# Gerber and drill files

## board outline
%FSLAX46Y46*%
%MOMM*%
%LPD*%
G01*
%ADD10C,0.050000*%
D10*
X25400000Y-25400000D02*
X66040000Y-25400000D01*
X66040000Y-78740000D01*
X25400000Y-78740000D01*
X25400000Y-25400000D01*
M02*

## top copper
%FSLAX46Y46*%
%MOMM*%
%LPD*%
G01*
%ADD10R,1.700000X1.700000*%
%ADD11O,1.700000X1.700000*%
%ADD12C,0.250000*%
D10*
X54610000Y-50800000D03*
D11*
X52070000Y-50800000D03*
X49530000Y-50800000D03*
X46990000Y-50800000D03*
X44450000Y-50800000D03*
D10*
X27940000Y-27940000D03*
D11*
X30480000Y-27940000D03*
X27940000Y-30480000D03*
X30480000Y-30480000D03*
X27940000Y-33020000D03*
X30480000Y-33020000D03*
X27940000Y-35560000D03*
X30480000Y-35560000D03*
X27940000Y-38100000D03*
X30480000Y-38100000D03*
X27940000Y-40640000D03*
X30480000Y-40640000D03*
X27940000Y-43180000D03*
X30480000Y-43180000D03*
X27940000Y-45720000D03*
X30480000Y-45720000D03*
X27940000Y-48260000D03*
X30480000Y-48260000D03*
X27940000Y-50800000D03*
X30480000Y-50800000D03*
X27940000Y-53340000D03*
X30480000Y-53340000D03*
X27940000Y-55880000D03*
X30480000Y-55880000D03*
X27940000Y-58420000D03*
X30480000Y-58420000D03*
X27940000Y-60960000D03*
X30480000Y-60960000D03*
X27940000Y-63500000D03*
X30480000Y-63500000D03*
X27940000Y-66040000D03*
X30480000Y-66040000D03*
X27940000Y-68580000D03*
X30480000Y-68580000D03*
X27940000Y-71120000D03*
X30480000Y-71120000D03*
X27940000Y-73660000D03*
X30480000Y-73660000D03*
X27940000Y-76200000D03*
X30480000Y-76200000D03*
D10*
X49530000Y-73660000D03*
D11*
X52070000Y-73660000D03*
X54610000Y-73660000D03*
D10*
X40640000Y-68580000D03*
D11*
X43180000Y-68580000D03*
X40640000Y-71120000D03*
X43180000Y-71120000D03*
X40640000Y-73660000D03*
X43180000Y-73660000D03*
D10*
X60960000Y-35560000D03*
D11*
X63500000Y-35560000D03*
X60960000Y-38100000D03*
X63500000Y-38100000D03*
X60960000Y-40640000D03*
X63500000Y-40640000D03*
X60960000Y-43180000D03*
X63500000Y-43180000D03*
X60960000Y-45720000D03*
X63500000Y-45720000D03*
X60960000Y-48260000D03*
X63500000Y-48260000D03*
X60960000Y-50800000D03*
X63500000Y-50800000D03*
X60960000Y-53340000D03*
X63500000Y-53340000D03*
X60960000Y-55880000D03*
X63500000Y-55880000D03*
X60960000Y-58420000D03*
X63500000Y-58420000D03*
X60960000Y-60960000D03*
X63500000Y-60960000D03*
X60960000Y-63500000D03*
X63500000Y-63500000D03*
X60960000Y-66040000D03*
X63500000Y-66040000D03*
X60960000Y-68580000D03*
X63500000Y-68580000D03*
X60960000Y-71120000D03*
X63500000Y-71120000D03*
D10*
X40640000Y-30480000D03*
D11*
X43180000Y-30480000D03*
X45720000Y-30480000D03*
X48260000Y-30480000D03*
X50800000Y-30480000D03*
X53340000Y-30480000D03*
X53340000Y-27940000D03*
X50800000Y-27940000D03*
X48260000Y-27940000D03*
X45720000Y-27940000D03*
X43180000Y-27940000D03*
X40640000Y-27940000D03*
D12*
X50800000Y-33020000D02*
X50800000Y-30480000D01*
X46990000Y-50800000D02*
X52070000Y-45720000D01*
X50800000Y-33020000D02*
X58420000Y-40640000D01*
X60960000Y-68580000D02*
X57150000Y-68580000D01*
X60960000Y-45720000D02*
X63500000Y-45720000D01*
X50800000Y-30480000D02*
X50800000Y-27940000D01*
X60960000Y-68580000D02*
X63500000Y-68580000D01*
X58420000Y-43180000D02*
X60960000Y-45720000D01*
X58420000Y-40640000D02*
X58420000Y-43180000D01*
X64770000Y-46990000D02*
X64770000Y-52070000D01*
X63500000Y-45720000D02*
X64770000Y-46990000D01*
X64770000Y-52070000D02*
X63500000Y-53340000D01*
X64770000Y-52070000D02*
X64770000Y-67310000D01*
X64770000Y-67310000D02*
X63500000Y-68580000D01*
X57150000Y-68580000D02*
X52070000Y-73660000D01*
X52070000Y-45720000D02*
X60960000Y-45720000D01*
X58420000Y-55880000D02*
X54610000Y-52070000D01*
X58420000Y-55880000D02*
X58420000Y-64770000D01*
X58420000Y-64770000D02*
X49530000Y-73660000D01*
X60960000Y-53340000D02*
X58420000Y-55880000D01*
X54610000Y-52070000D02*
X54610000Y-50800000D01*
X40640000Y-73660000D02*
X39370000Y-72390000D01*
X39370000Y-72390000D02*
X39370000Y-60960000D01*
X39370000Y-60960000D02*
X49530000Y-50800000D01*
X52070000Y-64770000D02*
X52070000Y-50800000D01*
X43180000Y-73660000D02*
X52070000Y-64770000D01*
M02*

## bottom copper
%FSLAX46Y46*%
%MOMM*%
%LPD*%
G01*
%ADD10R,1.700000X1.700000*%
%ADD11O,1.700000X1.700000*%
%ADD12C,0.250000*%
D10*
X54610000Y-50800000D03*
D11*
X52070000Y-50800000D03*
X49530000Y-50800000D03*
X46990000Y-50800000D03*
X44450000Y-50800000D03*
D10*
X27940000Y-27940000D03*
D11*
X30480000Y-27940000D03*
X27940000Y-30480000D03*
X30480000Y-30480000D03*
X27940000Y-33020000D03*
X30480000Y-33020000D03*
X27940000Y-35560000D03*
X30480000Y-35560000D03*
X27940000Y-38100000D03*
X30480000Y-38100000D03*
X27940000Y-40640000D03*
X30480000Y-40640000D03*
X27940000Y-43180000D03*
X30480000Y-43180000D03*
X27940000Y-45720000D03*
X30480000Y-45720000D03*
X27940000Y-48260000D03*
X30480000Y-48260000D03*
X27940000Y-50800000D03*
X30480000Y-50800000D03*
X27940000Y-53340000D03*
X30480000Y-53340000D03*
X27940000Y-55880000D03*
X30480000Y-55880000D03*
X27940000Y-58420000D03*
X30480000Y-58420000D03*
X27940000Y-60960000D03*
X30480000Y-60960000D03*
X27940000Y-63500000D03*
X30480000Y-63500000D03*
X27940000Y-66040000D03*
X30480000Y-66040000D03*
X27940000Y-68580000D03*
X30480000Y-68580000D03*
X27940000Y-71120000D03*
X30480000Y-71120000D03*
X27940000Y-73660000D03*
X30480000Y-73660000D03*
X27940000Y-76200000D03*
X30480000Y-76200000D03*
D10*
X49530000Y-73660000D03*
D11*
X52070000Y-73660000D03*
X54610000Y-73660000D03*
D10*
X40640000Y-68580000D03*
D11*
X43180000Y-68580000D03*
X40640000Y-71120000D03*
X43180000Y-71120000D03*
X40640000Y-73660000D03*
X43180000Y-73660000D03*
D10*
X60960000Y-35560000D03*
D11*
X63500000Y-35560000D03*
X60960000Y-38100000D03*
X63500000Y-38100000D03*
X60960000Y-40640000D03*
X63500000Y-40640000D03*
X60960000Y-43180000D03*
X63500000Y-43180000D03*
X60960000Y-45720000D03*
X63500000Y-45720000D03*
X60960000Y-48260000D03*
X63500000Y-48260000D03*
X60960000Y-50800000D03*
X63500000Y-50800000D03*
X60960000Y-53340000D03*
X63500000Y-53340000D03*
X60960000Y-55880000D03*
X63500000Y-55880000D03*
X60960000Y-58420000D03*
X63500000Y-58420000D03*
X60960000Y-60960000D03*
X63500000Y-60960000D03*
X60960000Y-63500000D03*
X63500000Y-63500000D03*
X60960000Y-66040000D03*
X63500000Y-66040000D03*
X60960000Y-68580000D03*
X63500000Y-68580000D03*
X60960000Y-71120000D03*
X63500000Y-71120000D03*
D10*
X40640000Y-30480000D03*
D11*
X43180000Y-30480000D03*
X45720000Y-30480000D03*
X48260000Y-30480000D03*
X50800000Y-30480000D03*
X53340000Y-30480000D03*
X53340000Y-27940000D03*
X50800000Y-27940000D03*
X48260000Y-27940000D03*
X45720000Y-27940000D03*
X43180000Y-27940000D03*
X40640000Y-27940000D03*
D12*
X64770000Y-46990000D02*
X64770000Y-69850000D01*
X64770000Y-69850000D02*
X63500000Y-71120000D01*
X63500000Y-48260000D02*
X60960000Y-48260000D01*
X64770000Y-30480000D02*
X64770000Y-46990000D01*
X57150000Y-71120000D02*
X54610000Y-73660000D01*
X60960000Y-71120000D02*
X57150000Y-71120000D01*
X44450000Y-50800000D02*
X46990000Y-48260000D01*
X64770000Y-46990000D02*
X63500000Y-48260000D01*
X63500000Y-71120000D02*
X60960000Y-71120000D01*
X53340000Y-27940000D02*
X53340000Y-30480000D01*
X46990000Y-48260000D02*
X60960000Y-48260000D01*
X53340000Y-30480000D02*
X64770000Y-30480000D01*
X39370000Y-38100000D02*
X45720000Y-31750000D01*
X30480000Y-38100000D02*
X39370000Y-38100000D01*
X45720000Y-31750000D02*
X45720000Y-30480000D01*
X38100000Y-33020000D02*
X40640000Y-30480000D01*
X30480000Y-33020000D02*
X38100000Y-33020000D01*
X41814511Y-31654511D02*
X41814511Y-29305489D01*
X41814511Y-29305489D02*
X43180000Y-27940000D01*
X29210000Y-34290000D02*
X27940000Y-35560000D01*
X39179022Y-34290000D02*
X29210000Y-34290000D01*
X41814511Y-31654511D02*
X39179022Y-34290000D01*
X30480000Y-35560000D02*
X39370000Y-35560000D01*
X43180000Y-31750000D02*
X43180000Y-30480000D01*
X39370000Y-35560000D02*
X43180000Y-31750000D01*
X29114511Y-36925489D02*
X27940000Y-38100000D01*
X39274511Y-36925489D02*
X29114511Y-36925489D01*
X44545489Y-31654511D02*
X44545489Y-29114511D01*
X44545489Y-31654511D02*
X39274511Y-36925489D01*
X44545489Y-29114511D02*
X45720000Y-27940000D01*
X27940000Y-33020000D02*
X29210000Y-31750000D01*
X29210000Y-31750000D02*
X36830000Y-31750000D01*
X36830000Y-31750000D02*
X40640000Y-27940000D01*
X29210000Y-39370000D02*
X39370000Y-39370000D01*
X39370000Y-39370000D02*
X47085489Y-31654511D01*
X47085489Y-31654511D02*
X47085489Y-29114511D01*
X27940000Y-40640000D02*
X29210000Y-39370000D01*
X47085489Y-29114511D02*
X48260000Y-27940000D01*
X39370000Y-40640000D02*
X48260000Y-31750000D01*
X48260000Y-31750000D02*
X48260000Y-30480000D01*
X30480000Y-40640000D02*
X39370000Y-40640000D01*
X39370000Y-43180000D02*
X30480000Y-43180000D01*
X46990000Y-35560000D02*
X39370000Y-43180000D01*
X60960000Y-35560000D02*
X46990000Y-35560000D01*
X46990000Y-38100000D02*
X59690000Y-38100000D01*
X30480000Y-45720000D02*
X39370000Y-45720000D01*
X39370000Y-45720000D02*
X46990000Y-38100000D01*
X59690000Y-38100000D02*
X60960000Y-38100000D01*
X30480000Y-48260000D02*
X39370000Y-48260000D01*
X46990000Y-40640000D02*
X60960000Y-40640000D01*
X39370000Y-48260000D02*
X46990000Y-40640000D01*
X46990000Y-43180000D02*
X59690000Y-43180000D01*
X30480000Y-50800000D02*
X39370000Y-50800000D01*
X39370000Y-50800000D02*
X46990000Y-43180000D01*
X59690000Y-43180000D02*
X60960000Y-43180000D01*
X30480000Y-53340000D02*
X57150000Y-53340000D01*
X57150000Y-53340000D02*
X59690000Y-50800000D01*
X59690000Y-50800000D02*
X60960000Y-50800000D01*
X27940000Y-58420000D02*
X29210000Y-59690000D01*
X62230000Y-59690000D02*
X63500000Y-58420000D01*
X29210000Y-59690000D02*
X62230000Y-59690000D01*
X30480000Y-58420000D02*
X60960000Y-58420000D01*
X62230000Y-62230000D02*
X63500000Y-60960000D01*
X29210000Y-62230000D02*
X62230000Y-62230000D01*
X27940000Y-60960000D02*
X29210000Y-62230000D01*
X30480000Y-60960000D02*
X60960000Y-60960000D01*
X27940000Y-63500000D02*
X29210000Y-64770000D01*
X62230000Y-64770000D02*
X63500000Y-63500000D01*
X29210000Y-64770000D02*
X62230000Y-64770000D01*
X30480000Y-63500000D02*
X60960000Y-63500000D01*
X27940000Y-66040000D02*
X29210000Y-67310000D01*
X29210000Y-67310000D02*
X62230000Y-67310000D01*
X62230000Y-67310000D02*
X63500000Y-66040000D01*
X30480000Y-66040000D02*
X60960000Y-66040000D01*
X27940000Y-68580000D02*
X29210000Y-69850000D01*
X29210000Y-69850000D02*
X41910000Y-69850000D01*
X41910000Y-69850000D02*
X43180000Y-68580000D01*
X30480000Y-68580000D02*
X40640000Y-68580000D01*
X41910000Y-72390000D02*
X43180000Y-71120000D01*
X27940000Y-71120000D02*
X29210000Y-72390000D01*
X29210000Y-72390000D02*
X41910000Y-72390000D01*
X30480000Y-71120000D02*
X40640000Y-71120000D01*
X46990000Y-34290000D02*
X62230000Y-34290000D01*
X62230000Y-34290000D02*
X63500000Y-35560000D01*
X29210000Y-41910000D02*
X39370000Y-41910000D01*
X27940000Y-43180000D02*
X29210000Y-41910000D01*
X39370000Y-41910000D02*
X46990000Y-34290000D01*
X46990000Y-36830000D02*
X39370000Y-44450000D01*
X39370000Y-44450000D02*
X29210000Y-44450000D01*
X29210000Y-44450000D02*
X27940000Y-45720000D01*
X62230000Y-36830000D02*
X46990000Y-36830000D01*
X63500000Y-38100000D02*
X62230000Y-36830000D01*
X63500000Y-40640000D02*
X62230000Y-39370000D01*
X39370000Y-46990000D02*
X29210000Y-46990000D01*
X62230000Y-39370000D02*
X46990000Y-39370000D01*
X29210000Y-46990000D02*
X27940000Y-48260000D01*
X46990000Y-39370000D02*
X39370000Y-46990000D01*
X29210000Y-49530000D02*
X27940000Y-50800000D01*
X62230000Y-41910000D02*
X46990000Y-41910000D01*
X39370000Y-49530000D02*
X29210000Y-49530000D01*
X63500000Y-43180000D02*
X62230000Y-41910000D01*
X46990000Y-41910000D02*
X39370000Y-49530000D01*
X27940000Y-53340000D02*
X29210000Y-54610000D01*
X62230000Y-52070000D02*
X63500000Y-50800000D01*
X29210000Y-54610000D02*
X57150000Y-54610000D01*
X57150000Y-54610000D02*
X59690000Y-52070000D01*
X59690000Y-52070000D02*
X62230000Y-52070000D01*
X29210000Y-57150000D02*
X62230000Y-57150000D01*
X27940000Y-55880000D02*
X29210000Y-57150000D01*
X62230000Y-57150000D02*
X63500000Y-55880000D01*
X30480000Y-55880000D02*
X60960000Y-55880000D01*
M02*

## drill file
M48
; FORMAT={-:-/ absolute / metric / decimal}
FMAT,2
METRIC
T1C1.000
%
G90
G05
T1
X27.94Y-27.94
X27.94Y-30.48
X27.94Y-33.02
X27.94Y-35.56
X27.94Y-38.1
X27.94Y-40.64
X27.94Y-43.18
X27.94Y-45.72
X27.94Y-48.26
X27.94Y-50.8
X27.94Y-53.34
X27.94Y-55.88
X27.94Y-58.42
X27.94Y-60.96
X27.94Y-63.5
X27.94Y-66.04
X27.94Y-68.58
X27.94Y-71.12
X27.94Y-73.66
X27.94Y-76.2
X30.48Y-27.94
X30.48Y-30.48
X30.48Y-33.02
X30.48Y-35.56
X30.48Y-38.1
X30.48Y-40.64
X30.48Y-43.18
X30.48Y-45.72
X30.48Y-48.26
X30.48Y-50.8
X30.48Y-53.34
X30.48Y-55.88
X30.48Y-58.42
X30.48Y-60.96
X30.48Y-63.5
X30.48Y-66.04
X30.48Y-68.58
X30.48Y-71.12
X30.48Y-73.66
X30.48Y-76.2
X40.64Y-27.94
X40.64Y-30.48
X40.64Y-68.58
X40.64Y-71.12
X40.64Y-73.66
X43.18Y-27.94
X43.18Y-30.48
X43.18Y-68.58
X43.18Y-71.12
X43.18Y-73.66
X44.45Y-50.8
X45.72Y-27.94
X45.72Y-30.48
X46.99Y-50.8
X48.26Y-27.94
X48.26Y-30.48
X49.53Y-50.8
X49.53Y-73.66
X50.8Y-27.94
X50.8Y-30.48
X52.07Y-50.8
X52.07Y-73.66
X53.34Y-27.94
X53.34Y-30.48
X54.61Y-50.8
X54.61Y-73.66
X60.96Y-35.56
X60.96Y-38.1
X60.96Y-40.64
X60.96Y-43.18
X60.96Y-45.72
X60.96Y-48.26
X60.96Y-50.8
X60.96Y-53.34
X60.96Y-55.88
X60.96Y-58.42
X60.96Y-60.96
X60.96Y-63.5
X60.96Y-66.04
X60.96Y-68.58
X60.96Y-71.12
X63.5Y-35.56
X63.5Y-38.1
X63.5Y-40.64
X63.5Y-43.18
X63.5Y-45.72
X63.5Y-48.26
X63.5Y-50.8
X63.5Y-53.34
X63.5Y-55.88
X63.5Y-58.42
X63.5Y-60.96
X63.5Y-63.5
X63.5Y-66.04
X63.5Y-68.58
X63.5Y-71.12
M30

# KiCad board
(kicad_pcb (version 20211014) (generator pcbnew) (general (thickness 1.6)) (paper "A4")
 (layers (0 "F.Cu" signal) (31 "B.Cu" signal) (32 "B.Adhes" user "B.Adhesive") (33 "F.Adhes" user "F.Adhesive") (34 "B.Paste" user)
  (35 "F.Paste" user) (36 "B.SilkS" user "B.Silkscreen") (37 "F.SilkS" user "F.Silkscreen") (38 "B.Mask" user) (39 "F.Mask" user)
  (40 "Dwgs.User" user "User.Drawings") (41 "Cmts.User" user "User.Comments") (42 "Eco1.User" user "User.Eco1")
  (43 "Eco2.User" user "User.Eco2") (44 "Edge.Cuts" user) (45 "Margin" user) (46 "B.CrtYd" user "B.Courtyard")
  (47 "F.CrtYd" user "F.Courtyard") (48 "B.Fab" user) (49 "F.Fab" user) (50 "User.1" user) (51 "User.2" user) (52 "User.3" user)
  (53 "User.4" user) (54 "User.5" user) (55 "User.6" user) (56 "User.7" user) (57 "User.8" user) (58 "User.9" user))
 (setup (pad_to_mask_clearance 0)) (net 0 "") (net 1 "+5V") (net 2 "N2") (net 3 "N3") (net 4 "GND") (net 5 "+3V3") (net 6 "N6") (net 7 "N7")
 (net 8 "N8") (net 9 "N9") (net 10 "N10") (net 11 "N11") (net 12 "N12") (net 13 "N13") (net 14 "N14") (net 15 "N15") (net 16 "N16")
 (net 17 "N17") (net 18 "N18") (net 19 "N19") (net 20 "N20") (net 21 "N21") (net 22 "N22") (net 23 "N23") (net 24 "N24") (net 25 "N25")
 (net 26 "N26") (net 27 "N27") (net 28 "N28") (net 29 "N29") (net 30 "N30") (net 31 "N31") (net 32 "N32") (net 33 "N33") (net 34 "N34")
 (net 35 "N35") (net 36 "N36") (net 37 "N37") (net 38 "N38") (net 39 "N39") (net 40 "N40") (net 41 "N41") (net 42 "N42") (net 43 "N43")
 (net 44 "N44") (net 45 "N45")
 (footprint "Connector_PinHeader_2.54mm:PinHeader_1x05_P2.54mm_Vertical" (layer "F.Cu") (at 54.61 50.8 -90)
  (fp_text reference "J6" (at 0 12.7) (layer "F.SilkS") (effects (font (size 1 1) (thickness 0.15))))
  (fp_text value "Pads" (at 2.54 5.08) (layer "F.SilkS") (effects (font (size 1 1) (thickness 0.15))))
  (pad "1" thru_hole rect (at 0 0 270) (size 1.7 1.7) (drill 1) (layers *.Cu *.Mask) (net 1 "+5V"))
  (pad "2" thru_hole oval (at 0 2.54 270) (size 1.7 1.7) (drill 1) (layers *.Cu *.Mask) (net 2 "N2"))
  (pad "3" thru_hole oval (at 0 5.08 270) (size 1.7 1.7) (drill 1) (layers *.Cu *.Mask) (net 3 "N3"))
  (pad "4" thru_hole oval (at 0 7.62 270) (size 1.7 1.7) (drill 1) (layers *.Cu *.Mask) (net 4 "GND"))
  (pad "5" thru_hole oval (at 0 10.16 270) (size 1.7 1.7) (drill 1) (layers *.Cu *.Mask) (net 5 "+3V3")))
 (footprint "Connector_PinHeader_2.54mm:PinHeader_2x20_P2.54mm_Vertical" (layer "F.Cu") (at 27.94 27.94)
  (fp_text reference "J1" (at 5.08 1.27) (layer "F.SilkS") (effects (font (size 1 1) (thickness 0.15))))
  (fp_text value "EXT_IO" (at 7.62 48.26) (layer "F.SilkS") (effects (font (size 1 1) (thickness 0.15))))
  (pad "1" thru_hole rect (at 0 0) (size 1.7 1.7) (drill 1) (layers *.Cu *.Mask) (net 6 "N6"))
  (pad "2" thru_hole oval (at 2.54 0) (size 1.7 1.7) (drill 1) (layers *.Cu *.Mask) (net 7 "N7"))
  (pad "3" thru_hole oval (at 0 2.54) (size 1.7 1.7) (drill 1) (layers *.Cu *.Mask) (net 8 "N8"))
  (pad "4" thru_hole oval (at 2.54 2.54) (size 1.7 1.7) (drill 1) (layers *.Cu *.Mask) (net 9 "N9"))
  (pad "5" thru_hole oval (at 0 5.08) (size 1.7 1.7) (drill 1) (layers *.Cu *.Mask) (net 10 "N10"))
  (pad "6" thru_hole oval (at 2.54 5.08) (size 1.7 1.7) (drill 1) (layers *.Cu *.Mask) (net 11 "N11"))
  (pad "7" thru_hole oval (at 0 7.62) (size 1.7 1.7) (drill 1) (layers *.Cu *.Mask) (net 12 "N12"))
  (pad "8" thru_hole oval (at 2.54 7.62) (size 1.7 1.7) (drill 1) (layers *.Cu *.Mask) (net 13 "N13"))
  (pad "9" thru_hole oval (at 0 10.16) (size 1.7 1.7) (drill 1) (layers *.Cu *.Mask) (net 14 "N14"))
  (pad "10" thru_hole oval (at 2.54 10.16) (size 1.7 1.7) (drill 1) (layers *.Cu *.Mask) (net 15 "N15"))
  (pad "11" thru_hole oval (at 0 12.7) (size 1.7 1.7) (drill 1) (layers *.Cu *.Mask) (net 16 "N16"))
  (pad "12" thru_hole oval (at 2.54 12.7) (size 1.7 1.7) (drill 1) (layers *.Cu *.Mask) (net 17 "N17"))
  (pad "13" thru_hole oval (at 0 15.24) (size 1.7 1.7) (drill 1) (layers *.Cu *.Mask) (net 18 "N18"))
  (pad "14" thru_hole oval (at 2.54 15.24) (size 1.7 1.7) (drill 1) (layers *.Cu *.Mask) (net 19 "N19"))
  (pad "15" thru_hole oval (at 0 17.78) (size 1.7 1.7) (drill 1) (layers *.Cu *.Mask) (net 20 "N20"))
  (pad "16" thru_hole oval (at 2.54 17.78) (size 1.7 1.7) (drill 1) (layers *.Cu *.Mask) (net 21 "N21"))
  (pad "17" thru_hole oval (at 0 20.32) (size 1.7 1.7) (drill 1) (layers *.Cu *.Mask) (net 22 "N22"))
  (pad "18" thru_hole oval (at 2.54 20.32) (size 1.7 1.7) (drill 1) (layers *.Cu *.Mask) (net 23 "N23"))
  (pad "19" thru_hole oval (at 0 22.86) (size 1.7 1.7) (drill 1) (layers *.Cu *.Mask) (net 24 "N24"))
  (pad "20" thru_hole oval (at 2.54 22.86) (size 1.7 1.7) (drill 1) (layers *.Cu *.Mask) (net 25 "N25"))
  (pad "21" thru_hole oval (at 0 25.4) (size 1.7 1.7) (drill 1) (layers *.Cu *.Mask) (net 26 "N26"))
  (pad "22" thru_hole oval (at 2.54 25.4) (size 1.7 1.7) (drill 1) (layers *.Cu *.Mask) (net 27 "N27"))
  (pad "23" thru_hole oval (at 0 27.94) (size 1.7 1.7) (drill 1) (layers *.Cu *.Mask) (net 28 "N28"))
  (pad "24" thru_hole oval (at 2.54 27.94) (size 1.7 1.7) (drill 1) (layers *.Cu *.Mask) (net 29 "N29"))
  (pad "25" thru_hole oval (at 0 30.48) (size 1.7 1.7) (drill 1) (layers *.Cu *.Mask) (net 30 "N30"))
  (pad "26" thru_hole oval (at 2.54 30.48) (size 1.7 1.7) (drill 1) (layers *.Cu *.Mask) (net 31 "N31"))
  (pad "27" thru_hole oval (at 0 33.02) (size 1.7 1.7) (drill 1) (layers *.Cu *.Mask) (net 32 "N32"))
  (pad "28" thru_hole oval (at 2.54 33.02) (size 1.7 1.7) (drill 1) (layers *.Cu *.Mask) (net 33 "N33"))
  (pad "29" thru_hole oval (at 0 35.56) (size 1.7 1.7) (drill 1) (layers *.Cu *.Mask) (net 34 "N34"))
  (pad "30" thru_hole oval (at 2.54 35.56) (size 1.7 1.7) (drill 1) (layers *.Cu *.Mask) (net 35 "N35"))
  (pad "31" thru_hole oval (at 0 38.1) (size 1.7 1.7) (drill 1) (layers *.Cu *.Mask) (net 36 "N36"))
  (pad "32" thru_hole oval (at 2.54 38.1) (size 1.7 1.7) (drill 1) (layers *.Cu *.Mask) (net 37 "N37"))
  (pad "33" thru_hole oval (at 0 40.64) (size 1.7 1.7) (drill 1) (layers *.Cu *.Mask) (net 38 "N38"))
  (pad "34" thru_hole oval (at 2.54 40.64) (size 1.7 1.7) (drill 1) (layers *.Cu *.Mask) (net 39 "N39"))
  (pad "35" thru_hole oval (at 0 43.18) (size 1.7 1.7) (drill 1) (layers *.Cu *.Mask) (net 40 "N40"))
  (pad "36" thru_hole oval (at 2.54 43.18) (size 1.7 1.7) (drill 1) (layers *.Cu *.Mask) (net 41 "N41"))
  (pad "37" thru_hole oval (at 0 45.72) (size 1.7 1.7) (drill 1) (layers *.Cu *.Mask) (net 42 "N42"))
  (pad "38" thru_hole oval (at 2.54 45.72) (size 1.7 1.7) (drill 1) (layers *.Cu *.Mask) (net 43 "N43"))
  (pad "39" thru_hole oval (at 0 48.26) (size 1.7 1.7) (drill 1) (layers *.Cu *.Mask) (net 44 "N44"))
  (pad "40" thru_hole oval (at 2.54 48.26) (size 1.7 1.7) (drill 1) (layers *.Cu *.Mask) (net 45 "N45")))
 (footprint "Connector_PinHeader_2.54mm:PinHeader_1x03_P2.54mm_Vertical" (layer "F.Cu") (at 49.53 73.66 90)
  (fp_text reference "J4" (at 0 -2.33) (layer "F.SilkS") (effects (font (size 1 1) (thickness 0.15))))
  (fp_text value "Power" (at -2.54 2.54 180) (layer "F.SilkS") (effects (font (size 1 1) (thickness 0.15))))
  (pad "1" thru_hole rect (at 0 0 90) (size 1.7 1.7) (drill 1) (layers *.Cu *.Mask) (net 1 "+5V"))
  (pad "2" thru_hole oval (at 0 2.54 90) (size 1.7 1.7) (drill 1) (layers *.Cu *.Mask) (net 4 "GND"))
  (pad "3" thru_hole oval (at 0 5.08 90) (size 1.7 1.7) (drill 1) (layers *.Cu *.Mask) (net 5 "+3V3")))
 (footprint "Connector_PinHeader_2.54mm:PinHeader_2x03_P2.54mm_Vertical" (layer "F.Cu") (at 40.64 68.58)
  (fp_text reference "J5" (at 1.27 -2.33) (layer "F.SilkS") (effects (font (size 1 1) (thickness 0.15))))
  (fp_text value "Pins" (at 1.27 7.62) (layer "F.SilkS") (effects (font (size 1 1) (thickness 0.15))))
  (pad "1" thru_hole rect (at 0 0) (size 1.7 1.7) (drill 1) (layers *.Cu *.Mask) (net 39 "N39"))
  (pad "2" thru_hole oval (at 2.54 0) (size 1.7 1.7) (drill 1) (layers *.Cu *.Mask) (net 38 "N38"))
  (pad "3" thru_hole oval (at 0 2.54) (size 1.7 1.7) (drill 1) (layers *.Cu *.Mask) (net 41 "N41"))
  (pad "4" thru_hole oval (at 2.54 2.54) (size 1.7 1.7) (drill 1) (layers *.Cu *.Mask) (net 40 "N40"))
  (pad "5" thru_hole oval (at 0 5.08) (size 1.7 1.7) (drill 1) (layers *.Cu *.Mask) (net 3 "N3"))
  (pad "6" thru_hole oval (at 2.54 5.08) (size 1.7 1.7) (drill 1) (layers *.Cu *.Mask) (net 2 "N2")))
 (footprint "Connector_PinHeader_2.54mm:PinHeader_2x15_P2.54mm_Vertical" (layer "F.Cu") (at 60.96 35.56)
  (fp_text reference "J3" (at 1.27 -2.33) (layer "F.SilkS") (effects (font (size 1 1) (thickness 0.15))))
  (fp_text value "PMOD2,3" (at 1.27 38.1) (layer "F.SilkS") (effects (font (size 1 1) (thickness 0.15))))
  (pad "1" thru_hole rect (at 0 0) (size 1.7 1.7) (drill 1) (layers *.Cu *.Mask) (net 19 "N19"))
  (pad "2" thru_hole oval (at 2.54 0) (size 1.7 1.7) (drill 1) (layers *.Cu *.Mask) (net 18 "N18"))
  (pad "3" thru_hole oval (at 0 2.54) (size 1.7 1.7) (drill 1) (layers *.Cu *.Mask) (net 21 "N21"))
  (pad "4" thru_hole oval (at 2.54 2.54) (size 1.7 1.7) (drill 1) (layers *.Cu *.Mask) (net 20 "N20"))
  (pad "5" thru_hole oval (at 0 5.08) (size 1.7 1.7) (drill 1) (layers *.Cu *.Mask) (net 23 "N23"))
  (pad "6" thru_hole oval (at 2.54 5.08) (size 1.7 1.7) (drill 1) (layers *.Cu *.Mask) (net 22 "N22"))
  (pad "7" thru_hole oval (at 0 7.62) (size 1.7 1.7) (drill 1) (layers *.Cu *.Mask) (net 25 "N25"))
  (pad "8" thru_hole oval (at 2.54 7.62) (size 1.7 1.7) (drill 1) (layers *.Cu *.Mask) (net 24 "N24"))
  (pad "9" thru_hole oval (at 0 10.16) (size 1.7 1.7) (drill 1) (layers *.Cu *.Mask) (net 4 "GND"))
  (pad "10" thru_hole oval (at 2.54 10.16) (size 1.7 1.7) (drill 1) (layers *.Cu *.Mask) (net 4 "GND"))
  (pad "11" thru_hole oval (at 0 12.7) (size 1.7 1.7) (drill 1) (layers *.Cu *.Mask) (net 5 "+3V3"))
  (pad "12" thru_hole oval (at 2.54 12.7) (size 1.7 1.7) (drill 1) (layers *.Cu *.Mask) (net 5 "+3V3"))
  (pad "13" thru_hole oval (at 0 15.24) (size 1.7 1.7) (drill 1) (layers *.Cu *.Mask) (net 27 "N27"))
  (pad "14" thru_hole oval (at 2.54 15.24) (size 1.7 1.7) (drill 1) (layers *.Cu *.Mask) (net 26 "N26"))
  (pad "15" thru_hole oval (at 0 17.78) (size 1.7 1.7) (drill 1) (layers *.Cu *.Mask) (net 1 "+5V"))
  (pad "16" thru_hole oval (at 2.54 17.78) (size 1.7 1.7) (drill 1) (layers *.Cu *.Mask) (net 4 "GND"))
  (pad "17" thru_hole oval (at 0 20.32) (size 1.7 1.7) (drill 1) (layers *.Cu *.Mask) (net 29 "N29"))
  (pad "18" thru_hole oval (at 2.54 20.32) (size 1.7 1.7) (drill 1) (layers *.Cu *.Mask) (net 28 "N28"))
  (pad "19" thru_hole oval (at 0 22.86) (size 1.7 1.7) (drill 1) (layers *.Cu *.Mask) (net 31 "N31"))
  (pad "20" thru_hole oval (at 2.54 22.86) (size 1.7 1.7) (drill 1) (layers *.Cu *.Mask) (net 30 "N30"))
  (pad "21" thru_hole oval (at 0 25.4) (size 1.7 1.7) (drill 1) (layers *.Cu *.Mask) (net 33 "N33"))
  (pad "22" thru_hole oval (at 2.54 25.4) (size 1.7 1.7) (drill 1) (layers *.Cu *.Mask) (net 32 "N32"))
  (pad "23" thru_hole oval (at 0 27.94) (size 1.7 1.7) (drill 1) (layers *.Cu *.Mask) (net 35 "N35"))
  (pad "24" thru_hole oval (at 2.54 27.94) (size 1.7 1.7) (drill 1) (layers *.Cu *.Mask) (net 34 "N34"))
  (pad "25" thru_hole oval (at 0 30.48) (size 1.7 1.7) (drill 1) (layers *.Cu *.Mask) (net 37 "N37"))
  (pad "26" thru_hole oval (at 2.54 30.48) (size 1.7 1.7) (drill 1) (layers *.Cu *.Mask) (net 36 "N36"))
  (pad "27" thru_hole oval (at 0 33.02) (size 1.7 1.7) (drill 1) (layers *.Cu *.Mask) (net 4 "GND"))
  (pad "28" thru_hole oval (at 2.54 33.02) (size 1.7 1.7) (drill 1) (layers *.Cu *.Mask) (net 4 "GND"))
  (pad "29" thru_hole oval (at 0 35.56) (size 1.7 1.7) (drill 1) (layers *.Cu *.Mask) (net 5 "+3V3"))
  (pad "30" thru_hole oval (at 2.54 35.56) (size 1.7 1.7) (drill 1) (layers *.Cu *.Mask) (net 5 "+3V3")))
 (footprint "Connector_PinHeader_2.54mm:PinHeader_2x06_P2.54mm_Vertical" (layer "F.Cu") (at 40.64 30.48 90)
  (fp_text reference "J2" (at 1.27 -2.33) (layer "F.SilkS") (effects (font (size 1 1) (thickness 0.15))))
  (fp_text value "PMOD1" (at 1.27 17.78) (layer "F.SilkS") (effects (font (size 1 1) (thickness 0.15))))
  (pad "1" thru_hole rect (at 0 0 90) (size 1.7 1.7) (drill 1) (layers *.Cu *.Mask) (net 11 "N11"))
  (pad "2" thru_hole oval (at 0 2.54 90) (size 1.7 1.7) (drill 1) (layers *.Cu *.Mask) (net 13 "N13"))
  (pad "3" thru_hole oval (at 0 5.08 90) (size 1.7 1.7) (drill 1) (layers *.Cu *.Mask) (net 15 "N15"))
  (pad "4" thru_hole oval (at 0 7.62 90) (size 1.7 1.7) (drill 1) (layers *.Cu *.Mask) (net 17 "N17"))
  (pad "5" thru_hole oval (at 0 10.16 90) (size 1.7 1.7) (drill 1) (layers *.Cu *.Mask) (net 4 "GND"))
  (pad "6" thru_hole oval (at 0 12.7 90) (size 1.7 1.7) (drill 1) (layers *.Cu *.Mask) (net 5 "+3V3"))
  (pad "7" thru_hole oval (at 2.54 12.7 90) (size 1.7 1.7) (drill 1) (layers *.Cu *.Mask) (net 5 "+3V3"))
  (pad "8" thru_hole oval (at 2.54 10.16 90) (size 1.7 1.7) (drill 1) (layers *.Cu *.Mask) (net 4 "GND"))
  (pad "9" thru_hole oval (at 2.54 7.62 90) (size 1.7 1.7) (drill 1) (layers *.Cu *.Mask) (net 16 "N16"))
  (pad "10" thru_hole oval (at 2.54 5.08 90) (size 1.7 1.7) (drill 1) (layers *.Cu *.Mask) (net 14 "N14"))
  (pad "11" thru_hole oval (at 2.54 2.54 90) (size 1.7 1.7) (drill 1) (layers *.Cu *.Mask) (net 12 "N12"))
  (pad "12" thru_hole oval (at 2.54 0 90) (size 1.7 1.7) (drill 1) (layers *.Cu *.Mask) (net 10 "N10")))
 (gr_rect (start 25.4 25.4) (end 66.04 78.74) (layer "Edge.Cuts") (width 0.05) (fill none))
 (segment (start 50.8 33.02) (end 50.8 30.48) (width 0.25) (layer "F.Cu") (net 4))
 (segment (start 46.99 50.8) (end 52.07 45.72) (width 0.25) (layer "F.Cu") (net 4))
 (segment (start 50.8 33.02) (end 58.42 40.64) (width 0.25) (layer "F.Cu") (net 4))
 (segment (start 60.96 68.58) (end 57.15 68.58) (width 0.25) (layer "F.Cu") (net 4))
 (segment (start 60.96 45.72) (end 63.5 45.72) (width 0.25) (layer "F.Cu") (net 4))
 (segment (start 50.8 30.48) (end 50.8 27.94) (width 0.25) (layer "F.Cu") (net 4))
 (segment (start 60.96 68.58) (end 63.5 68.58) (width 0.25) (layer "F.Cu") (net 4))
 (segment (start 58.42 43.18) (end 60.96 45.72) (width 0.25) (layer "F.Cu") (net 4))
 (segment (start 58.42 40.64) (end 58.42 43.18) (width 0.25) (layer "F.Cu") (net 4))
 (segment (start 64.77 46.99) (end 64.77 52.07) (width 0.25) (layer "F.Cu") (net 4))
 (segment (start 63.5 45.72) (end 64.77 46.99) (width 0.25) (layer "F.Cu") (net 4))
 (segment (start 64.77 52.07) (end 63.5 53.34) (width 0.25) (layer "F.Cu") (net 4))
 (segment (start 64.77 52.07) (end 64.77 67.31) (width 0.25) (layer "F.Cu") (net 4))
 (segment (start 64.77 67.31) (end 63.5 68.58) (width 0.25) (layer "F.Cu") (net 4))
 (segment (start 57.15 68.58) (end 52.07 73.66) (width 0.25) (layer "F.Cu") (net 4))
 (segment (start 52.07 45.72) (end 60.96 45.72) (width 0.25) (layer "F.Cu") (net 4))
 (segment (start 64.77 46.99) (end 64.77 69.85) (width 0.25) (layer "B.Cu") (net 5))
 (segment (start 64.77 69.85) (end 63.5 71.12) (width 0.25) (layer "B.Cu") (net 5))
 (segment (start 63.5 48.26) (end 60.96 48.26) (width 0.25) (layer "B.Cu") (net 5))
 (segment (start 64.77 30.48) (end 64.77 46.99) (width 0.25) (layer "B.Cu") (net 5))
 (segment (start 57.15 71.12) (end 54.61 73.66) (width 0.25) (layer "B.Cu") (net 5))
 (segment (start 60.96 71.12) (end 57.15 71.12) (width 0.25) (layer "B.Cu") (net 5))
 (segment (start 44.45 50.8) (end 46.99 48.26) (width 0.25) (layer "B.Cu") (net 5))
 (segment (start 64.77 46.99) (end 63.5 48.26) (width 0.25) (layer "B.Cu") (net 5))
 (segment (start 63.5 71.12) (end 60.96 71.12) (width 0.25) (layer "B.Cu") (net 5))
 (segment (start 53.34 27.94) (end 53.34 30.48) (width 0.25) (layer "B.Cu") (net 5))
 (segment (start 46.99 48.26) (end 60.96 48.26) (width 0.25) (layer "B.Cu") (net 5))
 (segment (start 53.34 30.48) (end 64.77 30.48) (width 0.25) (layer "B.Cu") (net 5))
 (segment (start 58.42 55.88) (end 54.61 52.07) (width 0.25) (layer "F.Cu") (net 1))
 (segment (start 58.42 55.88) (end 58.42 64.77) (width 0.25) (layer "F.Cu") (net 1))
 (segment (start 58.42 64.77) (end 49.53 73.66) (width 0.25) (layer "F.Cu") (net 1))
 (segment (start 60.96 53.34) (end 58.42 55.88) (width 0.25) (layer "F.Cu") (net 1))
 (segment (start 54.61 52.07) (end 54.61 50.8) (width 0.25) (layer "F.Cu") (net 1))
 (segment (start 39.37 38.1) (end 45.72 31.75) (width 0.25) (layer "B.Cu") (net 15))
 (segment (start 30.48 38.1) (end 39.37 38.1) (width 0.25) (layer "B.Cu") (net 15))
 (segment (start 45.72 31.75) (end 45.72 30.48) (width 0.25) (layer "B.Cu") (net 15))
 (segment (start 38.1 33.02) (end 40.64 30.48) (width 0.25) (layer "B.Cu") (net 11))
 (segment (start 30.48 33.02) (end 38.1 33.02) (width 0.25) (layer "B.Cu") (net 11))
 (segment (start 41.814511 31.654511) (end 41.814511 29.305489) (width 0.25) (layer "B.Cu") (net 12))
 (segment (start 41.814511 29.305489) (end 43.18 27.94) (width 0.25) (layer "B.Cu") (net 12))
 (segment (start 29.21 34.29) (end 27.94 35.56) (width 0.25) (layer "B.Cu") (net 12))
 (segment (start 39.179022 34.29) (end 29.21 34.29) (width 0.25) (layer "B.Cu") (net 12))
 (segment (start 41.814511 31.654511) (end 39.179022 34.29) (width 0.25) (layer "B.Cu") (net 12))
 (segment (start 30.48 35.56) (end 39.37 35.56) (width 0.25) (layer "B.Cu") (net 13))
 (segment (start 43.18 31.75) (end 43.18 30.48) (width 0.25) (layer "B.Cu") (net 13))
 (segment (start 39.37 35.56) (end 43.18 31.75) (width 0.25) (layer "B.Cu") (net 13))
 (segment (start 29.114511 36.925489) (end 27.94 38.1) (width 0.25) (layer "B.Cu") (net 14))
 (segment (start 39.274511 36.925489) (end 29.114511 36.925489) (width 0.25) (layer "B.Cu") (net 14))
 (segment (start 44.545489 31.654511) (end 44.545489 29.114511) (width 0.25) (layer "B.Cu") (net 14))
 (segment (start 44.545489 31.654511) (end 39.274511 36.925489) (width 0.25) (layer "B.Cu") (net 14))
 (segment (start 44.545489 29.114511) (end 45.72 27.94) (width 0.25) (layer "B.Cu") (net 14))
 (segment (start 27.94 33.02) (end 29.21 31.75) (width 0.25) (layer "B.Cu") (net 10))
 (segment (start 29.21 31.75) (end 36.83 31.75) (width 0.25) (layer "B.Cu") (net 10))
 (segment (start 36.83 31.75) (end 40.64 27.94) (width 0.25) (layer "B.Cu") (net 10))
 (segment (start 29.21 39.37) (end 39.37 39.37) (width 0.25) (layer "B.Cu") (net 16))
 (segment (start 39.37 39.37) (end 47.085489 31.654511) (width 0.25) (layer "B.Cu") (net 16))
 (segment (start 47.085489 31.654511) (end 47.085489 29.114511) (width 0.25) (layer "B.Cu") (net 16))
 (segment (start 27.94 40.64) (end 29.21 39.37) (width 0.25) (layer "B.Cu") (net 16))
 (segment (start 47.085489 29.114511) (end 48.26 27.94) (width 0.25) (layer "B.Cu") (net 16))
 (segment (start 39.37 40.64) (end 48.26 31.75) (width 0.25) (layer "B.Cu") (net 17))
 (segment (start 48.26 31.75) (end 48.26 30.48) (width 0.25) (layer "B.Cu") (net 17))
 (segment (start 30.48 40.64) (end 39.37 40.64) (width 0.25) (layer "B.Cu") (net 17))
 (segment (start 39.37 43.18) (end 30.48 43.18) (width 0.25) (layer "B.Cu") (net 19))
 (segment (start 46.99 35.56) (end 39.37 43.18) (width 0.25) (layer "B.Cu") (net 19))
 (segment (start 60.96 35.56) (end 46.99 35.56) (width 0.25) (layer "B.Cu") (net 19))
 (segment (start 46.99 38.1) (end 59.69 38.1) (width 0.25) (layer "B.Cu") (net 21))
 (segment (start 30.48 45.72) (end 39.37 45.72) (width 0.25) (layer "B.Cu") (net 21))
 (segment (start 39.37 45.72) (end 46.99 38.1) (width 0.25) (layer "B.Cu") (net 21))
 (segment (start 59.69 38.1) (end 60.96 38.1) (width 0.25) (layer "B.Cu") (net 21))
 (segment (start 30.48 48.26) (end 39.37 48.26) (width 0.25) (layer "B.Cu") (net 23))
 (segment (start 46.99 40.64) (end 60.96 40.64) (width 0.25) (layer "B.Cu") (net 23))
 (segment (start 39.37 48.26) (end 46.99 40.64) (width 0.25) (layer "B.Cu") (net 23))
 (segment (start 46.99 43.18) (end 59.69 43.18) (width 0.25) (layer "B.Cu") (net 25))
 (segment (start 30.48 50.8) (end 39.37 50.8) (width 0.25) (layer "B.Cu") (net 25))
 (segment (start 39.37 50.8) (end 46.99 43.18) (width 0.25) (layer "B.Cu") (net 25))
 (segment (start 59.69 43.18) (end 60.96 43.18) (width 0.25) (layer "B.Cu") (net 25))
 (segment (start 30.48 53.34) (end 57.15 53.34) (width 0.25) (layer "B.Cu") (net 27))
 (segment (start 57.15 53.34) (end 59.69 50.8) (width 0.25) (layer "B.Cu") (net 27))
 (segment (start 59.69 50.8) (end 60.96 50.8) (width 0.25) (layer "B.Cu") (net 27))
 (segment (start 27.94 58.42) (end 29.21 59.69) (width 0.25) (layer "B.Cu") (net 30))
 (segment (start 62.23 59.69) (end 63.5 58.42) (width 0.25) (layer "B.Cu") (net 30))
 (segment (start 29.21 59.69) (end 62.23 59.69) (width 0.25) (layer "B.Cu") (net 30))
 (segment (start 30.48 58.42) (end 60.96 58.42) (width 0.25) (layer "B.Cu") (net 31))
 (segment (start 62.23 62.23) (end 63.5 60.96) (width 0.25) (layer "B.Cu") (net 32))
 (segment (start 29.21 62.23) (end 62.23 62.23) (width 0.25) (layer "B.Cu") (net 32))
 (segment (start 27.94 60.96) (end 29.21 62.23) (width 0.25) (layer "B.Cu") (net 32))
 (segment (start 30.48 60.96) (end 60.96 60.96) (width 0.25) (layer "B.Cu") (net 33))
 (segment (start 27.94 63.5) (end 29.21 64.77) (width 0.25) (layer "B.Cu") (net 34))
 (segment (start 62.23 64.77) (end 63.5 63.5) (width 0.25) (layer "B.Cu") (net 34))
 (segment (start 29.21 64.77) (end 62.23 64.77) (width 0.25) (layer "B.Cu") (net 34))
 (segment (start 30.48 63.5) (end 60.96 63.5) (width 0.25) (layer "B.Cu") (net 35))
 (segment (start 27.94 66.04) (end 29.21 67.31) (width 0.25) (layer "B.Cu") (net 36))
 (segment (start 29.21 67.31) (end 62.23 67.31) (width 0.25) (layer "B.Cu") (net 36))
 (segment (start 62.23 67.31) (end 63.5 66.04) (width 0.25) (layer "B.Cu") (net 36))
 (segment (start 30.48 66.04) (end 60.96 66.04) (width 0.25) (layer "B.Cu") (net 37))
 (segment (start 27.94 68.58) (end 29.21 69.85) (width 0.25) (layer "B.Cu") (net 38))
 (segment (start 29.21 69.85) (end 41.91 69.85) (width 0.25) (layer "B.Cu") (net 38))
 (segment (start 41.91 69.85) (end 43.18 68.58) (width 0.25) (layer "B.Cu") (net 38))
 (segment (start 30.48 68.58) (end 40.64 68.58) (width 0.25) (layer "B.Cu") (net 39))
 (segment (start 41.91 72.39) (end 43.18 71.12) (width 0.25) (layer "B.Cu") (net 40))
 (segment (start 27.94 71.12) (end 29.21 72.39) (width 0.25) (layer "B.Cu") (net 40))
 (segment (start 29.21 72.39) (end 41.91 72.39) (width 0.25) (layer "B.Cu") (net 40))
 (segment (start 30.48 71.12) (end 40.64 71.12) (width 0.25) (layer "B.Cu") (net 41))
 (segment (start 46.99 34.29) (end 62.23 34.29) (width 0.25) (layer "B.Cu") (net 18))
 (segment (start 62.23 34.29) (end 63.5 35.56) (width 0.25) (layer "B.Cu") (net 18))
 (segment (start 29.21 41.91) (end 39.37 41.91) (width 0.25) (layer "B.Cu") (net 18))
 (segment (start 27.94 43.18) (end 29.21 41.91) (width 0.25) (layer "B.Cu") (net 18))
 (segment (start 39.37 41.91) (end 46.99 34.29) (width 0.25) (layer "B.Cu") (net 18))
 (segment (start 46.99 36.83) (end 39.37 44.45) (width 0.25) (layer "B.Cu") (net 20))
 (segment (start 39.37 44.45) (end 29.21 44.45) (width 0.25) (layer "B.Cu") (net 20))
 (segment (start 29.21 44.45) (end 27.94 45.72) (width 0.25) (layer "B.Cu") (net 20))
 (segment (start 62.23 36.83) (end 46.99 36.83) (width 0.25) (layer "B.Cu") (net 20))
 (segment (start 63.5 38.1) (end 62.23 36.83) (width 0.25) (layer "B.Cu") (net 20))
 (segment (start 63.5 40.64) (end 62.23 39.37) (width 0.25) (layer "B.Cu") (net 22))
 (segment (start 39.37 46.99) (end 29.21 46.99) (width 0.25) (layer "B.Cu") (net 22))
 (segment (start 62.23 39.37) (end 46.99 39.37) (width 0.25) (layer "B.Cu") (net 22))
 (segment (start 29.21 46.99) (end 27.94 48.26) (width 0.25) (layer "B.Cu") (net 22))
 (segment (start 46.99 39.37) (end 39.37 46.99) (width 0.25) (layer "B.Cu") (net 22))
 (segment (start 29.21 49.53) (end 27.94 50.8) (width 0.25) (layer "B.Cu") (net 24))
 (segment (start 62.23 41.91) (end 46.99 41.91) (width 0.25) (layer "B.Cu") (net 24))
 (segment (start 39.37 49.53) (end 29.21 49.53) (width 0.25) (layer "B.Cu") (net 24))
 (segment (start 63.5 43.18) (end 62.23 41.91) (width 0.25) (layer "B.Cu") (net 24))
 (segment (start 46.99 41.91) (end 39.37 49.53) (width 0.25) (layer "B.Cu") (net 24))
 (segment (start 27.94 53.34) (end 29.21 54.61) (width 0.25) (layer "B.Cu") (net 26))
 (segment (start 62.23 52.07) (end 63.5 50.8) (width 0.25) (layer "B.Cu") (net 26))
 (segment (start 29.21 54.61) (end 57.15 54.61) (width 0.25) (layer "B.Cu") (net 26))
 (segment (start 57.15 54.61) (end 59.69 52.07) (width 0.25) (layer "B.Cu") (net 26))
 (segment (start 59.69 52.07) (end 62.23 52.07) (width 0.25) (layer "B.Cu") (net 26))
 (segment (start 29.21 57.15) (end 62.23 57.15) (width 0.25) (layer "B.Cu") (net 28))
 (segment (start 27.94 55.88) (end 29.21 57.15) (width 0.25) (layer "B.Cu") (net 28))
 (segment (start 62.23 57.15) (end 63.5 55.88) (width 0.25) (layer "B.Cu") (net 28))
 (segment (start 30.48 55.88) (end 60.96 55.88) (width 0.25) (layer "B.Cu") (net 29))
 (segment (start 40.64 73.66) (end 39.37 72.39) (width 0.25) (layer "F.Cu") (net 3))
 (segment (start 39.37 72.39) (end 39.37 60.96) (width 0.25) (layer "F.Cu") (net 3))
 (segment (start 39.37 60.96) (end 49.53 50.8) (width 0.25) (layer "F.Cu") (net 3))
 (segment (start 52.07 64.77) (end 52.07 50.8) (width 0.25) (layer "F.Cu") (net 2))
 (segment (start 43.18 73.66) (end 52.07 64.77) (width 0.25) (layer "F.Cu") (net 2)))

